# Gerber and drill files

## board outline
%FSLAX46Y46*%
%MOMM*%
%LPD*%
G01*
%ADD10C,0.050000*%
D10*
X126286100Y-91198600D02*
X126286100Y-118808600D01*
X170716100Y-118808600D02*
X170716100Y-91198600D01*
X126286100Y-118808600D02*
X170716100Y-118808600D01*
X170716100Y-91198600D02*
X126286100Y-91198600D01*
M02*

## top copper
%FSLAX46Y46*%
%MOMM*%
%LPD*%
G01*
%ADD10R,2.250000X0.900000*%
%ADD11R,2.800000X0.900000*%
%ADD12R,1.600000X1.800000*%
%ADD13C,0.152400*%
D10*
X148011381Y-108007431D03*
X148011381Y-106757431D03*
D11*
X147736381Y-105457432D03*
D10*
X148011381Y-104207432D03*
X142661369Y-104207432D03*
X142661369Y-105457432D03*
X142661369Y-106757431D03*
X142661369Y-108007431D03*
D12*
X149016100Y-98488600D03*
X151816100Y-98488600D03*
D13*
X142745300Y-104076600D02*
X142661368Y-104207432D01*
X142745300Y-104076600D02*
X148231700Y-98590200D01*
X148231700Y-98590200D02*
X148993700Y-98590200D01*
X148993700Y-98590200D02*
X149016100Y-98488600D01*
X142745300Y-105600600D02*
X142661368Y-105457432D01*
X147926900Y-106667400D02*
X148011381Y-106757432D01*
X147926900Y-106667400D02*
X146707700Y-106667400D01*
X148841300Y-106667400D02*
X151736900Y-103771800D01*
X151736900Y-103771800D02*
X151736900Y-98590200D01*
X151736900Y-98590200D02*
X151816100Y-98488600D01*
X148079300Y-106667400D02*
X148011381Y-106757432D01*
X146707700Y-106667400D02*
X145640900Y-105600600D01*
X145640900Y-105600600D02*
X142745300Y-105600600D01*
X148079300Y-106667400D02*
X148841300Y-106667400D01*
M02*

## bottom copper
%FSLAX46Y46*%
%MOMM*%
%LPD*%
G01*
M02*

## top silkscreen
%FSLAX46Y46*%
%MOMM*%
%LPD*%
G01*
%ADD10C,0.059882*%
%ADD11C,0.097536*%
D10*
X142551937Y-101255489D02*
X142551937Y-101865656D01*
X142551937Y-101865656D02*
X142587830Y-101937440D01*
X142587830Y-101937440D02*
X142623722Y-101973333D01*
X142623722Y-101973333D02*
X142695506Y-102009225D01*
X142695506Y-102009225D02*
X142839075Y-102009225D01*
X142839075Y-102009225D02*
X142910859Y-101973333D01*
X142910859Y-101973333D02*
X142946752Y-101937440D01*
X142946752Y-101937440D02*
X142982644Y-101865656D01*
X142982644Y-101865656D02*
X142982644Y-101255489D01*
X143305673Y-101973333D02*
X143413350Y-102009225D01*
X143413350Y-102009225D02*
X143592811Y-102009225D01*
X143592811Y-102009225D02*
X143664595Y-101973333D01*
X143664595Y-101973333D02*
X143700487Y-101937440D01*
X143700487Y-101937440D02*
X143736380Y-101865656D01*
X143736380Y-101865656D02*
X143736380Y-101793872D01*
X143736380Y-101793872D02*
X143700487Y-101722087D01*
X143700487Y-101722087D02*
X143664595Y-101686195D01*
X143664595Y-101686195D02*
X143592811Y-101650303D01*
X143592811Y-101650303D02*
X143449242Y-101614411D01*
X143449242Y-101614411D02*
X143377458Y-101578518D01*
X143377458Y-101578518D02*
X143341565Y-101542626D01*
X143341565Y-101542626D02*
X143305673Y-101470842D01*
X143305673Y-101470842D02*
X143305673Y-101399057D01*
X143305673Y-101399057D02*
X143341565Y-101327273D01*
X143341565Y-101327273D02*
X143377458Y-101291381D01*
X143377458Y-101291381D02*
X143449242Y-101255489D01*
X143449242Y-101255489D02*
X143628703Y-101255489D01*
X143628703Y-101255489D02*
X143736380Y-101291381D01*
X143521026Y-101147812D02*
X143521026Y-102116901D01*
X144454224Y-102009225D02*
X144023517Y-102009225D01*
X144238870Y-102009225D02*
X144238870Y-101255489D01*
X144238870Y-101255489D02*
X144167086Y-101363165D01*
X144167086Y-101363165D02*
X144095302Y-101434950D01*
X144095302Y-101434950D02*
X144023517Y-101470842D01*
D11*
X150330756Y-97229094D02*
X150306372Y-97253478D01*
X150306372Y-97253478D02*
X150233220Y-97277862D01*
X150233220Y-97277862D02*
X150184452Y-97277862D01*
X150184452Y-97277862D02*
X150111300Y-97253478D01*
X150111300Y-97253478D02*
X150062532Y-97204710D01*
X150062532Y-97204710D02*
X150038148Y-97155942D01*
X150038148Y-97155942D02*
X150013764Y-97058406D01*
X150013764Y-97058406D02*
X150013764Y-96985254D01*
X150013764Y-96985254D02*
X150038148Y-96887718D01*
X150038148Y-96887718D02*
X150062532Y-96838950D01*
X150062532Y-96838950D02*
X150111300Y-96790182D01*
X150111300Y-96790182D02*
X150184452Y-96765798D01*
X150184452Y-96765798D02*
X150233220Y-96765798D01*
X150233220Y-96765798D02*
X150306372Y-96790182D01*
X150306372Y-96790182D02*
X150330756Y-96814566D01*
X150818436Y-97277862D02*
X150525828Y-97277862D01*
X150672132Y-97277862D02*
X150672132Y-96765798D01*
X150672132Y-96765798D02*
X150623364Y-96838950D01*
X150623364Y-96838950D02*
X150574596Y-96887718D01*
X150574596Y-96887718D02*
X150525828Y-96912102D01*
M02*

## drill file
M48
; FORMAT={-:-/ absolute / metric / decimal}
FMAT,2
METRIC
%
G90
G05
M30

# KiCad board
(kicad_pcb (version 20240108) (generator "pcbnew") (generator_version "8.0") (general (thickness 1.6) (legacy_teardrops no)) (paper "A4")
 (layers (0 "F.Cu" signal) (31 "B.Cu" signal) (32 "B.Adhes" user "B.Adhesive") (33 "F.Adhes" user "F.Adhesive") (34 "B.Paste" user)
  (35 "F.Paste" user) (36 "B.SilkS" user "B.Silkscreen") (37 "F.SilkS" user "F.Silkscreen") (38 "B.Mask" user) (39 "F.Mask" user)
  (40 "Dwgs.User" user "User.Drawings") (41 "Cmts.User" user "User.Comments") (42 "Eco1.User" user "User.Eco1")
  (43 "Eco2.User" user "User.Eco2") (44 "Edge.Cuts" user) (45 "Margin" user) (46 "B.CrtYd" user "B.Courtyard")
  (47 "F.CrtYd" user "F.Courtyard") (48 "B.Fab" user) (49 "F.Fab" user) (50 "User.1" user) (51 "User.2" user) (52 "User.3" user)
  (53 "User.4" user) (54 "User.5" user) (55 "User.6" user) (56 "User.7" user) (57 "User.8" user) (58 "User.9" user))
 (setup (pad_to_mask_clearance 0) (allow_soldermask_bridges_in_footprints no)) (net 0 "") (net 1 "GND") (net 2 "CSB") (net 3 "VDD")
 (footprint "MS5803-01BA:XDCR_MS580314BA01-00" (layer "F.Cu") (at 145.3361 106.1086)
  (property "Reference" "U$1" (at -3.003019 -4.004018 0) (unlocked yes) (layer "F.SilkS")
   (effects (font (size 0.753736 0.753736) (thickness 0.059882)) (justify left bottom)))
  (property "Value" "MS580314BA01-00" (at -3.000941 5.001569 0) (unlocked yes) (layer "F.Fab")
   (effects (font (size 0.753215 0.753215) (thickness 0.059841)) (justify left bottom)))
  (pad "1" smd rect (at 2.675281 1.898831) (size 2.25 0.9) (layers "F.Cu" "F.Paste" "F.Mask") (solder_mask_margin 0.1016)
   (thermal_bridge_angle 0))
  (pad "2" smd rect (at 2.675281 0.648831) (size 2.25 0.9) (layers "F.Cu" "F.Paste" "F.Mask") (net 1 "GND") (solder_mask_margin 0.1016)
   (thermal_bridge_angle 0))
  (pad "3" smd rect (at 2.400281 -0.651168) (size 2.8 0.9) (layers "F.Cu" "F.Paste" "F.Mask") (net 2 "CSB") (solder_mask_margin 0.1016)
   (thermal_bridge_angle 0))
  (pad "4" smd rect (at 2.675281 -1.901168) (size 2.25 0.9) (layers "F.Cu" "F.Paste" "F.Mask") (solder_mask_margin 0.1016)
   (thermal_bridge_angle 0))
  (pad "5" smd rect (at -2.674731 -1.901168) (size 2.25 0.9) (layers "F.Cu" "F.Paste" "F.Mask") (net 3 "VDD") (solder_mask_margin 0.1016)
   (thermal_bridge_angle 0))
  (pad "6" smd rect (at -2.674731 -0.651168) (size 2.25 0.9) (layers "F.Cu" "F.Paste" "F.Mask") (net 1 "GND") (solder_mask_margin 0.1016)
   (thermal_bridge_angle 0))
  (pad "7" smd rect (at -2.674731 0.648831) (size 2.25 0.9) (layers "F.Cu" "F.Paste" "F.Mask") (solder_mask_margin 0.1016)
   (thermal_bridge_angle 0))
  (pad "8" smd rect (at -2.674731 1.898831) (size 2.25 0.9) (layers "F.Cu" "F.Paste" "F.Mask") (solder_mask_margin 0.1016)
   (thermal_bridge_angle 0)))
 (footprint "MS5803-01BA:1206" (layer "F.Cu") (at 150.4161 98.4886)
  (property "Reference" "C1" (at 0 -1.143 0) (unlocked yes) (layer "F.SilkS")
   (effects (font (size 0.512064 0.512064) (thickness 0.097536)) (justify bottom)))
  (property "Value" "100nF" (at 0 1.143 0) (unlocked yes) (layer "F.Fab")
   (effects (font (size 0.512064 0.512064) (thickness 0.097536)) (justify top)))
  (pad "1" smd rect (at -1.4 0) (size 1.6 1.8) (layers "F.Cu" "F.Paste" "F.Mask") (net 3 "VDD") (solder_mask_margin 0.1016)
   (thermal_bridge_angle 0))
  (pad "2" smd rect (at 1.4 0) (size 1.6 1.8) (layers "F.Cu" "F.Paste" "F.Mask") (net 1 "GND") (solder_mask_margin 0.1016)
   (thermal_bridge_angle 0)))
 (gr_line (start 126.2861 91.1986) (end 126.2861 118.8086) (stroke (width 0.05) (type solid)) (layer "Edge.Cuts"))
 (gr_line (start 170.7161 118.8086) (end 170.7161 91.1986) (stroke (width 0.05) (type solid)) (layer "Edge.Cuts"))
 (gr_line (start 126.2861 118.8086) (end 170.7161 118.8086) (stroke (width 0.05) (type solid)) (layer "Edge.Cuts"))
 (gr_line (start 170.7161 91.1986) (end 126.2861 91.1986) (stroke (width 0.05) (type solid)) (layer "Edge.Cuts"))
 (segment (start 142.7453 104.0766) (end 142.661368 104.207432) (width 0.1524) (layer "F.Cu") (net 3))
 (segment (start 142.7453 104.0766) (end 148.2317 98.5902) (width 0.1524) (layer "F.Cu") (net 3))
 (segment (start 148.2317 98.5902) (end 148.9937 98.5902) (width 0.1524) (layer "F.Cu") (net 3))
 (segment (start 148.9937 98.5902) (end 149.0161 98.4886) (width 0.1524) (layer "F.Cu") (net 3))
 (segment (start 142.7453 105.6006) (end 142.661368 105.457432) (width 0.1524) (layer "F.Cu") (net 1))
 (segment (start 147.9269 106.6674) (end 148.011381 106.757432) (width 0.1524) (layer "F.Cu") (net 1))
 (segment (start 147.9269 106.6674) (end 146.7077 106.6674) (width 0.1524) (layer "F.Cu") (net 1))
 (segment (start 148.8413 106.6674) (end 151.7369 103.7718) (width 0.1524) (layer "F.Cu") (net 1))
 (segment (start 151.7369 103.7718) (end 151.7369 98.5902) (width 0.1524) (layer "F.Cu") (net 1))
 (segment (start 151.7369 98.5902) (end 151.8161 98.4886) (width 0.1524) (layer "F.Cu") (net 1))
 (segment (start 148.0793 106.6674) (end 148.011381 106.757432) (width 0.1524) (layer "F.Cu") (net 1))
 (segment (start 146.7077 106.6674) (end 145.6409 105.6006) (width 0.1524) (layer "F.Cu") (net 1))
 (segment (start 145.6409 105.6006) (end 142.7453 105.6006) (width 0.1524) (layer "F.Cu") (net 1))
 (segment (start 148.0793 106.6674) (end 148.8413 106.6674) (width 0.1524) (layer "F.Cu") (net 1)))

